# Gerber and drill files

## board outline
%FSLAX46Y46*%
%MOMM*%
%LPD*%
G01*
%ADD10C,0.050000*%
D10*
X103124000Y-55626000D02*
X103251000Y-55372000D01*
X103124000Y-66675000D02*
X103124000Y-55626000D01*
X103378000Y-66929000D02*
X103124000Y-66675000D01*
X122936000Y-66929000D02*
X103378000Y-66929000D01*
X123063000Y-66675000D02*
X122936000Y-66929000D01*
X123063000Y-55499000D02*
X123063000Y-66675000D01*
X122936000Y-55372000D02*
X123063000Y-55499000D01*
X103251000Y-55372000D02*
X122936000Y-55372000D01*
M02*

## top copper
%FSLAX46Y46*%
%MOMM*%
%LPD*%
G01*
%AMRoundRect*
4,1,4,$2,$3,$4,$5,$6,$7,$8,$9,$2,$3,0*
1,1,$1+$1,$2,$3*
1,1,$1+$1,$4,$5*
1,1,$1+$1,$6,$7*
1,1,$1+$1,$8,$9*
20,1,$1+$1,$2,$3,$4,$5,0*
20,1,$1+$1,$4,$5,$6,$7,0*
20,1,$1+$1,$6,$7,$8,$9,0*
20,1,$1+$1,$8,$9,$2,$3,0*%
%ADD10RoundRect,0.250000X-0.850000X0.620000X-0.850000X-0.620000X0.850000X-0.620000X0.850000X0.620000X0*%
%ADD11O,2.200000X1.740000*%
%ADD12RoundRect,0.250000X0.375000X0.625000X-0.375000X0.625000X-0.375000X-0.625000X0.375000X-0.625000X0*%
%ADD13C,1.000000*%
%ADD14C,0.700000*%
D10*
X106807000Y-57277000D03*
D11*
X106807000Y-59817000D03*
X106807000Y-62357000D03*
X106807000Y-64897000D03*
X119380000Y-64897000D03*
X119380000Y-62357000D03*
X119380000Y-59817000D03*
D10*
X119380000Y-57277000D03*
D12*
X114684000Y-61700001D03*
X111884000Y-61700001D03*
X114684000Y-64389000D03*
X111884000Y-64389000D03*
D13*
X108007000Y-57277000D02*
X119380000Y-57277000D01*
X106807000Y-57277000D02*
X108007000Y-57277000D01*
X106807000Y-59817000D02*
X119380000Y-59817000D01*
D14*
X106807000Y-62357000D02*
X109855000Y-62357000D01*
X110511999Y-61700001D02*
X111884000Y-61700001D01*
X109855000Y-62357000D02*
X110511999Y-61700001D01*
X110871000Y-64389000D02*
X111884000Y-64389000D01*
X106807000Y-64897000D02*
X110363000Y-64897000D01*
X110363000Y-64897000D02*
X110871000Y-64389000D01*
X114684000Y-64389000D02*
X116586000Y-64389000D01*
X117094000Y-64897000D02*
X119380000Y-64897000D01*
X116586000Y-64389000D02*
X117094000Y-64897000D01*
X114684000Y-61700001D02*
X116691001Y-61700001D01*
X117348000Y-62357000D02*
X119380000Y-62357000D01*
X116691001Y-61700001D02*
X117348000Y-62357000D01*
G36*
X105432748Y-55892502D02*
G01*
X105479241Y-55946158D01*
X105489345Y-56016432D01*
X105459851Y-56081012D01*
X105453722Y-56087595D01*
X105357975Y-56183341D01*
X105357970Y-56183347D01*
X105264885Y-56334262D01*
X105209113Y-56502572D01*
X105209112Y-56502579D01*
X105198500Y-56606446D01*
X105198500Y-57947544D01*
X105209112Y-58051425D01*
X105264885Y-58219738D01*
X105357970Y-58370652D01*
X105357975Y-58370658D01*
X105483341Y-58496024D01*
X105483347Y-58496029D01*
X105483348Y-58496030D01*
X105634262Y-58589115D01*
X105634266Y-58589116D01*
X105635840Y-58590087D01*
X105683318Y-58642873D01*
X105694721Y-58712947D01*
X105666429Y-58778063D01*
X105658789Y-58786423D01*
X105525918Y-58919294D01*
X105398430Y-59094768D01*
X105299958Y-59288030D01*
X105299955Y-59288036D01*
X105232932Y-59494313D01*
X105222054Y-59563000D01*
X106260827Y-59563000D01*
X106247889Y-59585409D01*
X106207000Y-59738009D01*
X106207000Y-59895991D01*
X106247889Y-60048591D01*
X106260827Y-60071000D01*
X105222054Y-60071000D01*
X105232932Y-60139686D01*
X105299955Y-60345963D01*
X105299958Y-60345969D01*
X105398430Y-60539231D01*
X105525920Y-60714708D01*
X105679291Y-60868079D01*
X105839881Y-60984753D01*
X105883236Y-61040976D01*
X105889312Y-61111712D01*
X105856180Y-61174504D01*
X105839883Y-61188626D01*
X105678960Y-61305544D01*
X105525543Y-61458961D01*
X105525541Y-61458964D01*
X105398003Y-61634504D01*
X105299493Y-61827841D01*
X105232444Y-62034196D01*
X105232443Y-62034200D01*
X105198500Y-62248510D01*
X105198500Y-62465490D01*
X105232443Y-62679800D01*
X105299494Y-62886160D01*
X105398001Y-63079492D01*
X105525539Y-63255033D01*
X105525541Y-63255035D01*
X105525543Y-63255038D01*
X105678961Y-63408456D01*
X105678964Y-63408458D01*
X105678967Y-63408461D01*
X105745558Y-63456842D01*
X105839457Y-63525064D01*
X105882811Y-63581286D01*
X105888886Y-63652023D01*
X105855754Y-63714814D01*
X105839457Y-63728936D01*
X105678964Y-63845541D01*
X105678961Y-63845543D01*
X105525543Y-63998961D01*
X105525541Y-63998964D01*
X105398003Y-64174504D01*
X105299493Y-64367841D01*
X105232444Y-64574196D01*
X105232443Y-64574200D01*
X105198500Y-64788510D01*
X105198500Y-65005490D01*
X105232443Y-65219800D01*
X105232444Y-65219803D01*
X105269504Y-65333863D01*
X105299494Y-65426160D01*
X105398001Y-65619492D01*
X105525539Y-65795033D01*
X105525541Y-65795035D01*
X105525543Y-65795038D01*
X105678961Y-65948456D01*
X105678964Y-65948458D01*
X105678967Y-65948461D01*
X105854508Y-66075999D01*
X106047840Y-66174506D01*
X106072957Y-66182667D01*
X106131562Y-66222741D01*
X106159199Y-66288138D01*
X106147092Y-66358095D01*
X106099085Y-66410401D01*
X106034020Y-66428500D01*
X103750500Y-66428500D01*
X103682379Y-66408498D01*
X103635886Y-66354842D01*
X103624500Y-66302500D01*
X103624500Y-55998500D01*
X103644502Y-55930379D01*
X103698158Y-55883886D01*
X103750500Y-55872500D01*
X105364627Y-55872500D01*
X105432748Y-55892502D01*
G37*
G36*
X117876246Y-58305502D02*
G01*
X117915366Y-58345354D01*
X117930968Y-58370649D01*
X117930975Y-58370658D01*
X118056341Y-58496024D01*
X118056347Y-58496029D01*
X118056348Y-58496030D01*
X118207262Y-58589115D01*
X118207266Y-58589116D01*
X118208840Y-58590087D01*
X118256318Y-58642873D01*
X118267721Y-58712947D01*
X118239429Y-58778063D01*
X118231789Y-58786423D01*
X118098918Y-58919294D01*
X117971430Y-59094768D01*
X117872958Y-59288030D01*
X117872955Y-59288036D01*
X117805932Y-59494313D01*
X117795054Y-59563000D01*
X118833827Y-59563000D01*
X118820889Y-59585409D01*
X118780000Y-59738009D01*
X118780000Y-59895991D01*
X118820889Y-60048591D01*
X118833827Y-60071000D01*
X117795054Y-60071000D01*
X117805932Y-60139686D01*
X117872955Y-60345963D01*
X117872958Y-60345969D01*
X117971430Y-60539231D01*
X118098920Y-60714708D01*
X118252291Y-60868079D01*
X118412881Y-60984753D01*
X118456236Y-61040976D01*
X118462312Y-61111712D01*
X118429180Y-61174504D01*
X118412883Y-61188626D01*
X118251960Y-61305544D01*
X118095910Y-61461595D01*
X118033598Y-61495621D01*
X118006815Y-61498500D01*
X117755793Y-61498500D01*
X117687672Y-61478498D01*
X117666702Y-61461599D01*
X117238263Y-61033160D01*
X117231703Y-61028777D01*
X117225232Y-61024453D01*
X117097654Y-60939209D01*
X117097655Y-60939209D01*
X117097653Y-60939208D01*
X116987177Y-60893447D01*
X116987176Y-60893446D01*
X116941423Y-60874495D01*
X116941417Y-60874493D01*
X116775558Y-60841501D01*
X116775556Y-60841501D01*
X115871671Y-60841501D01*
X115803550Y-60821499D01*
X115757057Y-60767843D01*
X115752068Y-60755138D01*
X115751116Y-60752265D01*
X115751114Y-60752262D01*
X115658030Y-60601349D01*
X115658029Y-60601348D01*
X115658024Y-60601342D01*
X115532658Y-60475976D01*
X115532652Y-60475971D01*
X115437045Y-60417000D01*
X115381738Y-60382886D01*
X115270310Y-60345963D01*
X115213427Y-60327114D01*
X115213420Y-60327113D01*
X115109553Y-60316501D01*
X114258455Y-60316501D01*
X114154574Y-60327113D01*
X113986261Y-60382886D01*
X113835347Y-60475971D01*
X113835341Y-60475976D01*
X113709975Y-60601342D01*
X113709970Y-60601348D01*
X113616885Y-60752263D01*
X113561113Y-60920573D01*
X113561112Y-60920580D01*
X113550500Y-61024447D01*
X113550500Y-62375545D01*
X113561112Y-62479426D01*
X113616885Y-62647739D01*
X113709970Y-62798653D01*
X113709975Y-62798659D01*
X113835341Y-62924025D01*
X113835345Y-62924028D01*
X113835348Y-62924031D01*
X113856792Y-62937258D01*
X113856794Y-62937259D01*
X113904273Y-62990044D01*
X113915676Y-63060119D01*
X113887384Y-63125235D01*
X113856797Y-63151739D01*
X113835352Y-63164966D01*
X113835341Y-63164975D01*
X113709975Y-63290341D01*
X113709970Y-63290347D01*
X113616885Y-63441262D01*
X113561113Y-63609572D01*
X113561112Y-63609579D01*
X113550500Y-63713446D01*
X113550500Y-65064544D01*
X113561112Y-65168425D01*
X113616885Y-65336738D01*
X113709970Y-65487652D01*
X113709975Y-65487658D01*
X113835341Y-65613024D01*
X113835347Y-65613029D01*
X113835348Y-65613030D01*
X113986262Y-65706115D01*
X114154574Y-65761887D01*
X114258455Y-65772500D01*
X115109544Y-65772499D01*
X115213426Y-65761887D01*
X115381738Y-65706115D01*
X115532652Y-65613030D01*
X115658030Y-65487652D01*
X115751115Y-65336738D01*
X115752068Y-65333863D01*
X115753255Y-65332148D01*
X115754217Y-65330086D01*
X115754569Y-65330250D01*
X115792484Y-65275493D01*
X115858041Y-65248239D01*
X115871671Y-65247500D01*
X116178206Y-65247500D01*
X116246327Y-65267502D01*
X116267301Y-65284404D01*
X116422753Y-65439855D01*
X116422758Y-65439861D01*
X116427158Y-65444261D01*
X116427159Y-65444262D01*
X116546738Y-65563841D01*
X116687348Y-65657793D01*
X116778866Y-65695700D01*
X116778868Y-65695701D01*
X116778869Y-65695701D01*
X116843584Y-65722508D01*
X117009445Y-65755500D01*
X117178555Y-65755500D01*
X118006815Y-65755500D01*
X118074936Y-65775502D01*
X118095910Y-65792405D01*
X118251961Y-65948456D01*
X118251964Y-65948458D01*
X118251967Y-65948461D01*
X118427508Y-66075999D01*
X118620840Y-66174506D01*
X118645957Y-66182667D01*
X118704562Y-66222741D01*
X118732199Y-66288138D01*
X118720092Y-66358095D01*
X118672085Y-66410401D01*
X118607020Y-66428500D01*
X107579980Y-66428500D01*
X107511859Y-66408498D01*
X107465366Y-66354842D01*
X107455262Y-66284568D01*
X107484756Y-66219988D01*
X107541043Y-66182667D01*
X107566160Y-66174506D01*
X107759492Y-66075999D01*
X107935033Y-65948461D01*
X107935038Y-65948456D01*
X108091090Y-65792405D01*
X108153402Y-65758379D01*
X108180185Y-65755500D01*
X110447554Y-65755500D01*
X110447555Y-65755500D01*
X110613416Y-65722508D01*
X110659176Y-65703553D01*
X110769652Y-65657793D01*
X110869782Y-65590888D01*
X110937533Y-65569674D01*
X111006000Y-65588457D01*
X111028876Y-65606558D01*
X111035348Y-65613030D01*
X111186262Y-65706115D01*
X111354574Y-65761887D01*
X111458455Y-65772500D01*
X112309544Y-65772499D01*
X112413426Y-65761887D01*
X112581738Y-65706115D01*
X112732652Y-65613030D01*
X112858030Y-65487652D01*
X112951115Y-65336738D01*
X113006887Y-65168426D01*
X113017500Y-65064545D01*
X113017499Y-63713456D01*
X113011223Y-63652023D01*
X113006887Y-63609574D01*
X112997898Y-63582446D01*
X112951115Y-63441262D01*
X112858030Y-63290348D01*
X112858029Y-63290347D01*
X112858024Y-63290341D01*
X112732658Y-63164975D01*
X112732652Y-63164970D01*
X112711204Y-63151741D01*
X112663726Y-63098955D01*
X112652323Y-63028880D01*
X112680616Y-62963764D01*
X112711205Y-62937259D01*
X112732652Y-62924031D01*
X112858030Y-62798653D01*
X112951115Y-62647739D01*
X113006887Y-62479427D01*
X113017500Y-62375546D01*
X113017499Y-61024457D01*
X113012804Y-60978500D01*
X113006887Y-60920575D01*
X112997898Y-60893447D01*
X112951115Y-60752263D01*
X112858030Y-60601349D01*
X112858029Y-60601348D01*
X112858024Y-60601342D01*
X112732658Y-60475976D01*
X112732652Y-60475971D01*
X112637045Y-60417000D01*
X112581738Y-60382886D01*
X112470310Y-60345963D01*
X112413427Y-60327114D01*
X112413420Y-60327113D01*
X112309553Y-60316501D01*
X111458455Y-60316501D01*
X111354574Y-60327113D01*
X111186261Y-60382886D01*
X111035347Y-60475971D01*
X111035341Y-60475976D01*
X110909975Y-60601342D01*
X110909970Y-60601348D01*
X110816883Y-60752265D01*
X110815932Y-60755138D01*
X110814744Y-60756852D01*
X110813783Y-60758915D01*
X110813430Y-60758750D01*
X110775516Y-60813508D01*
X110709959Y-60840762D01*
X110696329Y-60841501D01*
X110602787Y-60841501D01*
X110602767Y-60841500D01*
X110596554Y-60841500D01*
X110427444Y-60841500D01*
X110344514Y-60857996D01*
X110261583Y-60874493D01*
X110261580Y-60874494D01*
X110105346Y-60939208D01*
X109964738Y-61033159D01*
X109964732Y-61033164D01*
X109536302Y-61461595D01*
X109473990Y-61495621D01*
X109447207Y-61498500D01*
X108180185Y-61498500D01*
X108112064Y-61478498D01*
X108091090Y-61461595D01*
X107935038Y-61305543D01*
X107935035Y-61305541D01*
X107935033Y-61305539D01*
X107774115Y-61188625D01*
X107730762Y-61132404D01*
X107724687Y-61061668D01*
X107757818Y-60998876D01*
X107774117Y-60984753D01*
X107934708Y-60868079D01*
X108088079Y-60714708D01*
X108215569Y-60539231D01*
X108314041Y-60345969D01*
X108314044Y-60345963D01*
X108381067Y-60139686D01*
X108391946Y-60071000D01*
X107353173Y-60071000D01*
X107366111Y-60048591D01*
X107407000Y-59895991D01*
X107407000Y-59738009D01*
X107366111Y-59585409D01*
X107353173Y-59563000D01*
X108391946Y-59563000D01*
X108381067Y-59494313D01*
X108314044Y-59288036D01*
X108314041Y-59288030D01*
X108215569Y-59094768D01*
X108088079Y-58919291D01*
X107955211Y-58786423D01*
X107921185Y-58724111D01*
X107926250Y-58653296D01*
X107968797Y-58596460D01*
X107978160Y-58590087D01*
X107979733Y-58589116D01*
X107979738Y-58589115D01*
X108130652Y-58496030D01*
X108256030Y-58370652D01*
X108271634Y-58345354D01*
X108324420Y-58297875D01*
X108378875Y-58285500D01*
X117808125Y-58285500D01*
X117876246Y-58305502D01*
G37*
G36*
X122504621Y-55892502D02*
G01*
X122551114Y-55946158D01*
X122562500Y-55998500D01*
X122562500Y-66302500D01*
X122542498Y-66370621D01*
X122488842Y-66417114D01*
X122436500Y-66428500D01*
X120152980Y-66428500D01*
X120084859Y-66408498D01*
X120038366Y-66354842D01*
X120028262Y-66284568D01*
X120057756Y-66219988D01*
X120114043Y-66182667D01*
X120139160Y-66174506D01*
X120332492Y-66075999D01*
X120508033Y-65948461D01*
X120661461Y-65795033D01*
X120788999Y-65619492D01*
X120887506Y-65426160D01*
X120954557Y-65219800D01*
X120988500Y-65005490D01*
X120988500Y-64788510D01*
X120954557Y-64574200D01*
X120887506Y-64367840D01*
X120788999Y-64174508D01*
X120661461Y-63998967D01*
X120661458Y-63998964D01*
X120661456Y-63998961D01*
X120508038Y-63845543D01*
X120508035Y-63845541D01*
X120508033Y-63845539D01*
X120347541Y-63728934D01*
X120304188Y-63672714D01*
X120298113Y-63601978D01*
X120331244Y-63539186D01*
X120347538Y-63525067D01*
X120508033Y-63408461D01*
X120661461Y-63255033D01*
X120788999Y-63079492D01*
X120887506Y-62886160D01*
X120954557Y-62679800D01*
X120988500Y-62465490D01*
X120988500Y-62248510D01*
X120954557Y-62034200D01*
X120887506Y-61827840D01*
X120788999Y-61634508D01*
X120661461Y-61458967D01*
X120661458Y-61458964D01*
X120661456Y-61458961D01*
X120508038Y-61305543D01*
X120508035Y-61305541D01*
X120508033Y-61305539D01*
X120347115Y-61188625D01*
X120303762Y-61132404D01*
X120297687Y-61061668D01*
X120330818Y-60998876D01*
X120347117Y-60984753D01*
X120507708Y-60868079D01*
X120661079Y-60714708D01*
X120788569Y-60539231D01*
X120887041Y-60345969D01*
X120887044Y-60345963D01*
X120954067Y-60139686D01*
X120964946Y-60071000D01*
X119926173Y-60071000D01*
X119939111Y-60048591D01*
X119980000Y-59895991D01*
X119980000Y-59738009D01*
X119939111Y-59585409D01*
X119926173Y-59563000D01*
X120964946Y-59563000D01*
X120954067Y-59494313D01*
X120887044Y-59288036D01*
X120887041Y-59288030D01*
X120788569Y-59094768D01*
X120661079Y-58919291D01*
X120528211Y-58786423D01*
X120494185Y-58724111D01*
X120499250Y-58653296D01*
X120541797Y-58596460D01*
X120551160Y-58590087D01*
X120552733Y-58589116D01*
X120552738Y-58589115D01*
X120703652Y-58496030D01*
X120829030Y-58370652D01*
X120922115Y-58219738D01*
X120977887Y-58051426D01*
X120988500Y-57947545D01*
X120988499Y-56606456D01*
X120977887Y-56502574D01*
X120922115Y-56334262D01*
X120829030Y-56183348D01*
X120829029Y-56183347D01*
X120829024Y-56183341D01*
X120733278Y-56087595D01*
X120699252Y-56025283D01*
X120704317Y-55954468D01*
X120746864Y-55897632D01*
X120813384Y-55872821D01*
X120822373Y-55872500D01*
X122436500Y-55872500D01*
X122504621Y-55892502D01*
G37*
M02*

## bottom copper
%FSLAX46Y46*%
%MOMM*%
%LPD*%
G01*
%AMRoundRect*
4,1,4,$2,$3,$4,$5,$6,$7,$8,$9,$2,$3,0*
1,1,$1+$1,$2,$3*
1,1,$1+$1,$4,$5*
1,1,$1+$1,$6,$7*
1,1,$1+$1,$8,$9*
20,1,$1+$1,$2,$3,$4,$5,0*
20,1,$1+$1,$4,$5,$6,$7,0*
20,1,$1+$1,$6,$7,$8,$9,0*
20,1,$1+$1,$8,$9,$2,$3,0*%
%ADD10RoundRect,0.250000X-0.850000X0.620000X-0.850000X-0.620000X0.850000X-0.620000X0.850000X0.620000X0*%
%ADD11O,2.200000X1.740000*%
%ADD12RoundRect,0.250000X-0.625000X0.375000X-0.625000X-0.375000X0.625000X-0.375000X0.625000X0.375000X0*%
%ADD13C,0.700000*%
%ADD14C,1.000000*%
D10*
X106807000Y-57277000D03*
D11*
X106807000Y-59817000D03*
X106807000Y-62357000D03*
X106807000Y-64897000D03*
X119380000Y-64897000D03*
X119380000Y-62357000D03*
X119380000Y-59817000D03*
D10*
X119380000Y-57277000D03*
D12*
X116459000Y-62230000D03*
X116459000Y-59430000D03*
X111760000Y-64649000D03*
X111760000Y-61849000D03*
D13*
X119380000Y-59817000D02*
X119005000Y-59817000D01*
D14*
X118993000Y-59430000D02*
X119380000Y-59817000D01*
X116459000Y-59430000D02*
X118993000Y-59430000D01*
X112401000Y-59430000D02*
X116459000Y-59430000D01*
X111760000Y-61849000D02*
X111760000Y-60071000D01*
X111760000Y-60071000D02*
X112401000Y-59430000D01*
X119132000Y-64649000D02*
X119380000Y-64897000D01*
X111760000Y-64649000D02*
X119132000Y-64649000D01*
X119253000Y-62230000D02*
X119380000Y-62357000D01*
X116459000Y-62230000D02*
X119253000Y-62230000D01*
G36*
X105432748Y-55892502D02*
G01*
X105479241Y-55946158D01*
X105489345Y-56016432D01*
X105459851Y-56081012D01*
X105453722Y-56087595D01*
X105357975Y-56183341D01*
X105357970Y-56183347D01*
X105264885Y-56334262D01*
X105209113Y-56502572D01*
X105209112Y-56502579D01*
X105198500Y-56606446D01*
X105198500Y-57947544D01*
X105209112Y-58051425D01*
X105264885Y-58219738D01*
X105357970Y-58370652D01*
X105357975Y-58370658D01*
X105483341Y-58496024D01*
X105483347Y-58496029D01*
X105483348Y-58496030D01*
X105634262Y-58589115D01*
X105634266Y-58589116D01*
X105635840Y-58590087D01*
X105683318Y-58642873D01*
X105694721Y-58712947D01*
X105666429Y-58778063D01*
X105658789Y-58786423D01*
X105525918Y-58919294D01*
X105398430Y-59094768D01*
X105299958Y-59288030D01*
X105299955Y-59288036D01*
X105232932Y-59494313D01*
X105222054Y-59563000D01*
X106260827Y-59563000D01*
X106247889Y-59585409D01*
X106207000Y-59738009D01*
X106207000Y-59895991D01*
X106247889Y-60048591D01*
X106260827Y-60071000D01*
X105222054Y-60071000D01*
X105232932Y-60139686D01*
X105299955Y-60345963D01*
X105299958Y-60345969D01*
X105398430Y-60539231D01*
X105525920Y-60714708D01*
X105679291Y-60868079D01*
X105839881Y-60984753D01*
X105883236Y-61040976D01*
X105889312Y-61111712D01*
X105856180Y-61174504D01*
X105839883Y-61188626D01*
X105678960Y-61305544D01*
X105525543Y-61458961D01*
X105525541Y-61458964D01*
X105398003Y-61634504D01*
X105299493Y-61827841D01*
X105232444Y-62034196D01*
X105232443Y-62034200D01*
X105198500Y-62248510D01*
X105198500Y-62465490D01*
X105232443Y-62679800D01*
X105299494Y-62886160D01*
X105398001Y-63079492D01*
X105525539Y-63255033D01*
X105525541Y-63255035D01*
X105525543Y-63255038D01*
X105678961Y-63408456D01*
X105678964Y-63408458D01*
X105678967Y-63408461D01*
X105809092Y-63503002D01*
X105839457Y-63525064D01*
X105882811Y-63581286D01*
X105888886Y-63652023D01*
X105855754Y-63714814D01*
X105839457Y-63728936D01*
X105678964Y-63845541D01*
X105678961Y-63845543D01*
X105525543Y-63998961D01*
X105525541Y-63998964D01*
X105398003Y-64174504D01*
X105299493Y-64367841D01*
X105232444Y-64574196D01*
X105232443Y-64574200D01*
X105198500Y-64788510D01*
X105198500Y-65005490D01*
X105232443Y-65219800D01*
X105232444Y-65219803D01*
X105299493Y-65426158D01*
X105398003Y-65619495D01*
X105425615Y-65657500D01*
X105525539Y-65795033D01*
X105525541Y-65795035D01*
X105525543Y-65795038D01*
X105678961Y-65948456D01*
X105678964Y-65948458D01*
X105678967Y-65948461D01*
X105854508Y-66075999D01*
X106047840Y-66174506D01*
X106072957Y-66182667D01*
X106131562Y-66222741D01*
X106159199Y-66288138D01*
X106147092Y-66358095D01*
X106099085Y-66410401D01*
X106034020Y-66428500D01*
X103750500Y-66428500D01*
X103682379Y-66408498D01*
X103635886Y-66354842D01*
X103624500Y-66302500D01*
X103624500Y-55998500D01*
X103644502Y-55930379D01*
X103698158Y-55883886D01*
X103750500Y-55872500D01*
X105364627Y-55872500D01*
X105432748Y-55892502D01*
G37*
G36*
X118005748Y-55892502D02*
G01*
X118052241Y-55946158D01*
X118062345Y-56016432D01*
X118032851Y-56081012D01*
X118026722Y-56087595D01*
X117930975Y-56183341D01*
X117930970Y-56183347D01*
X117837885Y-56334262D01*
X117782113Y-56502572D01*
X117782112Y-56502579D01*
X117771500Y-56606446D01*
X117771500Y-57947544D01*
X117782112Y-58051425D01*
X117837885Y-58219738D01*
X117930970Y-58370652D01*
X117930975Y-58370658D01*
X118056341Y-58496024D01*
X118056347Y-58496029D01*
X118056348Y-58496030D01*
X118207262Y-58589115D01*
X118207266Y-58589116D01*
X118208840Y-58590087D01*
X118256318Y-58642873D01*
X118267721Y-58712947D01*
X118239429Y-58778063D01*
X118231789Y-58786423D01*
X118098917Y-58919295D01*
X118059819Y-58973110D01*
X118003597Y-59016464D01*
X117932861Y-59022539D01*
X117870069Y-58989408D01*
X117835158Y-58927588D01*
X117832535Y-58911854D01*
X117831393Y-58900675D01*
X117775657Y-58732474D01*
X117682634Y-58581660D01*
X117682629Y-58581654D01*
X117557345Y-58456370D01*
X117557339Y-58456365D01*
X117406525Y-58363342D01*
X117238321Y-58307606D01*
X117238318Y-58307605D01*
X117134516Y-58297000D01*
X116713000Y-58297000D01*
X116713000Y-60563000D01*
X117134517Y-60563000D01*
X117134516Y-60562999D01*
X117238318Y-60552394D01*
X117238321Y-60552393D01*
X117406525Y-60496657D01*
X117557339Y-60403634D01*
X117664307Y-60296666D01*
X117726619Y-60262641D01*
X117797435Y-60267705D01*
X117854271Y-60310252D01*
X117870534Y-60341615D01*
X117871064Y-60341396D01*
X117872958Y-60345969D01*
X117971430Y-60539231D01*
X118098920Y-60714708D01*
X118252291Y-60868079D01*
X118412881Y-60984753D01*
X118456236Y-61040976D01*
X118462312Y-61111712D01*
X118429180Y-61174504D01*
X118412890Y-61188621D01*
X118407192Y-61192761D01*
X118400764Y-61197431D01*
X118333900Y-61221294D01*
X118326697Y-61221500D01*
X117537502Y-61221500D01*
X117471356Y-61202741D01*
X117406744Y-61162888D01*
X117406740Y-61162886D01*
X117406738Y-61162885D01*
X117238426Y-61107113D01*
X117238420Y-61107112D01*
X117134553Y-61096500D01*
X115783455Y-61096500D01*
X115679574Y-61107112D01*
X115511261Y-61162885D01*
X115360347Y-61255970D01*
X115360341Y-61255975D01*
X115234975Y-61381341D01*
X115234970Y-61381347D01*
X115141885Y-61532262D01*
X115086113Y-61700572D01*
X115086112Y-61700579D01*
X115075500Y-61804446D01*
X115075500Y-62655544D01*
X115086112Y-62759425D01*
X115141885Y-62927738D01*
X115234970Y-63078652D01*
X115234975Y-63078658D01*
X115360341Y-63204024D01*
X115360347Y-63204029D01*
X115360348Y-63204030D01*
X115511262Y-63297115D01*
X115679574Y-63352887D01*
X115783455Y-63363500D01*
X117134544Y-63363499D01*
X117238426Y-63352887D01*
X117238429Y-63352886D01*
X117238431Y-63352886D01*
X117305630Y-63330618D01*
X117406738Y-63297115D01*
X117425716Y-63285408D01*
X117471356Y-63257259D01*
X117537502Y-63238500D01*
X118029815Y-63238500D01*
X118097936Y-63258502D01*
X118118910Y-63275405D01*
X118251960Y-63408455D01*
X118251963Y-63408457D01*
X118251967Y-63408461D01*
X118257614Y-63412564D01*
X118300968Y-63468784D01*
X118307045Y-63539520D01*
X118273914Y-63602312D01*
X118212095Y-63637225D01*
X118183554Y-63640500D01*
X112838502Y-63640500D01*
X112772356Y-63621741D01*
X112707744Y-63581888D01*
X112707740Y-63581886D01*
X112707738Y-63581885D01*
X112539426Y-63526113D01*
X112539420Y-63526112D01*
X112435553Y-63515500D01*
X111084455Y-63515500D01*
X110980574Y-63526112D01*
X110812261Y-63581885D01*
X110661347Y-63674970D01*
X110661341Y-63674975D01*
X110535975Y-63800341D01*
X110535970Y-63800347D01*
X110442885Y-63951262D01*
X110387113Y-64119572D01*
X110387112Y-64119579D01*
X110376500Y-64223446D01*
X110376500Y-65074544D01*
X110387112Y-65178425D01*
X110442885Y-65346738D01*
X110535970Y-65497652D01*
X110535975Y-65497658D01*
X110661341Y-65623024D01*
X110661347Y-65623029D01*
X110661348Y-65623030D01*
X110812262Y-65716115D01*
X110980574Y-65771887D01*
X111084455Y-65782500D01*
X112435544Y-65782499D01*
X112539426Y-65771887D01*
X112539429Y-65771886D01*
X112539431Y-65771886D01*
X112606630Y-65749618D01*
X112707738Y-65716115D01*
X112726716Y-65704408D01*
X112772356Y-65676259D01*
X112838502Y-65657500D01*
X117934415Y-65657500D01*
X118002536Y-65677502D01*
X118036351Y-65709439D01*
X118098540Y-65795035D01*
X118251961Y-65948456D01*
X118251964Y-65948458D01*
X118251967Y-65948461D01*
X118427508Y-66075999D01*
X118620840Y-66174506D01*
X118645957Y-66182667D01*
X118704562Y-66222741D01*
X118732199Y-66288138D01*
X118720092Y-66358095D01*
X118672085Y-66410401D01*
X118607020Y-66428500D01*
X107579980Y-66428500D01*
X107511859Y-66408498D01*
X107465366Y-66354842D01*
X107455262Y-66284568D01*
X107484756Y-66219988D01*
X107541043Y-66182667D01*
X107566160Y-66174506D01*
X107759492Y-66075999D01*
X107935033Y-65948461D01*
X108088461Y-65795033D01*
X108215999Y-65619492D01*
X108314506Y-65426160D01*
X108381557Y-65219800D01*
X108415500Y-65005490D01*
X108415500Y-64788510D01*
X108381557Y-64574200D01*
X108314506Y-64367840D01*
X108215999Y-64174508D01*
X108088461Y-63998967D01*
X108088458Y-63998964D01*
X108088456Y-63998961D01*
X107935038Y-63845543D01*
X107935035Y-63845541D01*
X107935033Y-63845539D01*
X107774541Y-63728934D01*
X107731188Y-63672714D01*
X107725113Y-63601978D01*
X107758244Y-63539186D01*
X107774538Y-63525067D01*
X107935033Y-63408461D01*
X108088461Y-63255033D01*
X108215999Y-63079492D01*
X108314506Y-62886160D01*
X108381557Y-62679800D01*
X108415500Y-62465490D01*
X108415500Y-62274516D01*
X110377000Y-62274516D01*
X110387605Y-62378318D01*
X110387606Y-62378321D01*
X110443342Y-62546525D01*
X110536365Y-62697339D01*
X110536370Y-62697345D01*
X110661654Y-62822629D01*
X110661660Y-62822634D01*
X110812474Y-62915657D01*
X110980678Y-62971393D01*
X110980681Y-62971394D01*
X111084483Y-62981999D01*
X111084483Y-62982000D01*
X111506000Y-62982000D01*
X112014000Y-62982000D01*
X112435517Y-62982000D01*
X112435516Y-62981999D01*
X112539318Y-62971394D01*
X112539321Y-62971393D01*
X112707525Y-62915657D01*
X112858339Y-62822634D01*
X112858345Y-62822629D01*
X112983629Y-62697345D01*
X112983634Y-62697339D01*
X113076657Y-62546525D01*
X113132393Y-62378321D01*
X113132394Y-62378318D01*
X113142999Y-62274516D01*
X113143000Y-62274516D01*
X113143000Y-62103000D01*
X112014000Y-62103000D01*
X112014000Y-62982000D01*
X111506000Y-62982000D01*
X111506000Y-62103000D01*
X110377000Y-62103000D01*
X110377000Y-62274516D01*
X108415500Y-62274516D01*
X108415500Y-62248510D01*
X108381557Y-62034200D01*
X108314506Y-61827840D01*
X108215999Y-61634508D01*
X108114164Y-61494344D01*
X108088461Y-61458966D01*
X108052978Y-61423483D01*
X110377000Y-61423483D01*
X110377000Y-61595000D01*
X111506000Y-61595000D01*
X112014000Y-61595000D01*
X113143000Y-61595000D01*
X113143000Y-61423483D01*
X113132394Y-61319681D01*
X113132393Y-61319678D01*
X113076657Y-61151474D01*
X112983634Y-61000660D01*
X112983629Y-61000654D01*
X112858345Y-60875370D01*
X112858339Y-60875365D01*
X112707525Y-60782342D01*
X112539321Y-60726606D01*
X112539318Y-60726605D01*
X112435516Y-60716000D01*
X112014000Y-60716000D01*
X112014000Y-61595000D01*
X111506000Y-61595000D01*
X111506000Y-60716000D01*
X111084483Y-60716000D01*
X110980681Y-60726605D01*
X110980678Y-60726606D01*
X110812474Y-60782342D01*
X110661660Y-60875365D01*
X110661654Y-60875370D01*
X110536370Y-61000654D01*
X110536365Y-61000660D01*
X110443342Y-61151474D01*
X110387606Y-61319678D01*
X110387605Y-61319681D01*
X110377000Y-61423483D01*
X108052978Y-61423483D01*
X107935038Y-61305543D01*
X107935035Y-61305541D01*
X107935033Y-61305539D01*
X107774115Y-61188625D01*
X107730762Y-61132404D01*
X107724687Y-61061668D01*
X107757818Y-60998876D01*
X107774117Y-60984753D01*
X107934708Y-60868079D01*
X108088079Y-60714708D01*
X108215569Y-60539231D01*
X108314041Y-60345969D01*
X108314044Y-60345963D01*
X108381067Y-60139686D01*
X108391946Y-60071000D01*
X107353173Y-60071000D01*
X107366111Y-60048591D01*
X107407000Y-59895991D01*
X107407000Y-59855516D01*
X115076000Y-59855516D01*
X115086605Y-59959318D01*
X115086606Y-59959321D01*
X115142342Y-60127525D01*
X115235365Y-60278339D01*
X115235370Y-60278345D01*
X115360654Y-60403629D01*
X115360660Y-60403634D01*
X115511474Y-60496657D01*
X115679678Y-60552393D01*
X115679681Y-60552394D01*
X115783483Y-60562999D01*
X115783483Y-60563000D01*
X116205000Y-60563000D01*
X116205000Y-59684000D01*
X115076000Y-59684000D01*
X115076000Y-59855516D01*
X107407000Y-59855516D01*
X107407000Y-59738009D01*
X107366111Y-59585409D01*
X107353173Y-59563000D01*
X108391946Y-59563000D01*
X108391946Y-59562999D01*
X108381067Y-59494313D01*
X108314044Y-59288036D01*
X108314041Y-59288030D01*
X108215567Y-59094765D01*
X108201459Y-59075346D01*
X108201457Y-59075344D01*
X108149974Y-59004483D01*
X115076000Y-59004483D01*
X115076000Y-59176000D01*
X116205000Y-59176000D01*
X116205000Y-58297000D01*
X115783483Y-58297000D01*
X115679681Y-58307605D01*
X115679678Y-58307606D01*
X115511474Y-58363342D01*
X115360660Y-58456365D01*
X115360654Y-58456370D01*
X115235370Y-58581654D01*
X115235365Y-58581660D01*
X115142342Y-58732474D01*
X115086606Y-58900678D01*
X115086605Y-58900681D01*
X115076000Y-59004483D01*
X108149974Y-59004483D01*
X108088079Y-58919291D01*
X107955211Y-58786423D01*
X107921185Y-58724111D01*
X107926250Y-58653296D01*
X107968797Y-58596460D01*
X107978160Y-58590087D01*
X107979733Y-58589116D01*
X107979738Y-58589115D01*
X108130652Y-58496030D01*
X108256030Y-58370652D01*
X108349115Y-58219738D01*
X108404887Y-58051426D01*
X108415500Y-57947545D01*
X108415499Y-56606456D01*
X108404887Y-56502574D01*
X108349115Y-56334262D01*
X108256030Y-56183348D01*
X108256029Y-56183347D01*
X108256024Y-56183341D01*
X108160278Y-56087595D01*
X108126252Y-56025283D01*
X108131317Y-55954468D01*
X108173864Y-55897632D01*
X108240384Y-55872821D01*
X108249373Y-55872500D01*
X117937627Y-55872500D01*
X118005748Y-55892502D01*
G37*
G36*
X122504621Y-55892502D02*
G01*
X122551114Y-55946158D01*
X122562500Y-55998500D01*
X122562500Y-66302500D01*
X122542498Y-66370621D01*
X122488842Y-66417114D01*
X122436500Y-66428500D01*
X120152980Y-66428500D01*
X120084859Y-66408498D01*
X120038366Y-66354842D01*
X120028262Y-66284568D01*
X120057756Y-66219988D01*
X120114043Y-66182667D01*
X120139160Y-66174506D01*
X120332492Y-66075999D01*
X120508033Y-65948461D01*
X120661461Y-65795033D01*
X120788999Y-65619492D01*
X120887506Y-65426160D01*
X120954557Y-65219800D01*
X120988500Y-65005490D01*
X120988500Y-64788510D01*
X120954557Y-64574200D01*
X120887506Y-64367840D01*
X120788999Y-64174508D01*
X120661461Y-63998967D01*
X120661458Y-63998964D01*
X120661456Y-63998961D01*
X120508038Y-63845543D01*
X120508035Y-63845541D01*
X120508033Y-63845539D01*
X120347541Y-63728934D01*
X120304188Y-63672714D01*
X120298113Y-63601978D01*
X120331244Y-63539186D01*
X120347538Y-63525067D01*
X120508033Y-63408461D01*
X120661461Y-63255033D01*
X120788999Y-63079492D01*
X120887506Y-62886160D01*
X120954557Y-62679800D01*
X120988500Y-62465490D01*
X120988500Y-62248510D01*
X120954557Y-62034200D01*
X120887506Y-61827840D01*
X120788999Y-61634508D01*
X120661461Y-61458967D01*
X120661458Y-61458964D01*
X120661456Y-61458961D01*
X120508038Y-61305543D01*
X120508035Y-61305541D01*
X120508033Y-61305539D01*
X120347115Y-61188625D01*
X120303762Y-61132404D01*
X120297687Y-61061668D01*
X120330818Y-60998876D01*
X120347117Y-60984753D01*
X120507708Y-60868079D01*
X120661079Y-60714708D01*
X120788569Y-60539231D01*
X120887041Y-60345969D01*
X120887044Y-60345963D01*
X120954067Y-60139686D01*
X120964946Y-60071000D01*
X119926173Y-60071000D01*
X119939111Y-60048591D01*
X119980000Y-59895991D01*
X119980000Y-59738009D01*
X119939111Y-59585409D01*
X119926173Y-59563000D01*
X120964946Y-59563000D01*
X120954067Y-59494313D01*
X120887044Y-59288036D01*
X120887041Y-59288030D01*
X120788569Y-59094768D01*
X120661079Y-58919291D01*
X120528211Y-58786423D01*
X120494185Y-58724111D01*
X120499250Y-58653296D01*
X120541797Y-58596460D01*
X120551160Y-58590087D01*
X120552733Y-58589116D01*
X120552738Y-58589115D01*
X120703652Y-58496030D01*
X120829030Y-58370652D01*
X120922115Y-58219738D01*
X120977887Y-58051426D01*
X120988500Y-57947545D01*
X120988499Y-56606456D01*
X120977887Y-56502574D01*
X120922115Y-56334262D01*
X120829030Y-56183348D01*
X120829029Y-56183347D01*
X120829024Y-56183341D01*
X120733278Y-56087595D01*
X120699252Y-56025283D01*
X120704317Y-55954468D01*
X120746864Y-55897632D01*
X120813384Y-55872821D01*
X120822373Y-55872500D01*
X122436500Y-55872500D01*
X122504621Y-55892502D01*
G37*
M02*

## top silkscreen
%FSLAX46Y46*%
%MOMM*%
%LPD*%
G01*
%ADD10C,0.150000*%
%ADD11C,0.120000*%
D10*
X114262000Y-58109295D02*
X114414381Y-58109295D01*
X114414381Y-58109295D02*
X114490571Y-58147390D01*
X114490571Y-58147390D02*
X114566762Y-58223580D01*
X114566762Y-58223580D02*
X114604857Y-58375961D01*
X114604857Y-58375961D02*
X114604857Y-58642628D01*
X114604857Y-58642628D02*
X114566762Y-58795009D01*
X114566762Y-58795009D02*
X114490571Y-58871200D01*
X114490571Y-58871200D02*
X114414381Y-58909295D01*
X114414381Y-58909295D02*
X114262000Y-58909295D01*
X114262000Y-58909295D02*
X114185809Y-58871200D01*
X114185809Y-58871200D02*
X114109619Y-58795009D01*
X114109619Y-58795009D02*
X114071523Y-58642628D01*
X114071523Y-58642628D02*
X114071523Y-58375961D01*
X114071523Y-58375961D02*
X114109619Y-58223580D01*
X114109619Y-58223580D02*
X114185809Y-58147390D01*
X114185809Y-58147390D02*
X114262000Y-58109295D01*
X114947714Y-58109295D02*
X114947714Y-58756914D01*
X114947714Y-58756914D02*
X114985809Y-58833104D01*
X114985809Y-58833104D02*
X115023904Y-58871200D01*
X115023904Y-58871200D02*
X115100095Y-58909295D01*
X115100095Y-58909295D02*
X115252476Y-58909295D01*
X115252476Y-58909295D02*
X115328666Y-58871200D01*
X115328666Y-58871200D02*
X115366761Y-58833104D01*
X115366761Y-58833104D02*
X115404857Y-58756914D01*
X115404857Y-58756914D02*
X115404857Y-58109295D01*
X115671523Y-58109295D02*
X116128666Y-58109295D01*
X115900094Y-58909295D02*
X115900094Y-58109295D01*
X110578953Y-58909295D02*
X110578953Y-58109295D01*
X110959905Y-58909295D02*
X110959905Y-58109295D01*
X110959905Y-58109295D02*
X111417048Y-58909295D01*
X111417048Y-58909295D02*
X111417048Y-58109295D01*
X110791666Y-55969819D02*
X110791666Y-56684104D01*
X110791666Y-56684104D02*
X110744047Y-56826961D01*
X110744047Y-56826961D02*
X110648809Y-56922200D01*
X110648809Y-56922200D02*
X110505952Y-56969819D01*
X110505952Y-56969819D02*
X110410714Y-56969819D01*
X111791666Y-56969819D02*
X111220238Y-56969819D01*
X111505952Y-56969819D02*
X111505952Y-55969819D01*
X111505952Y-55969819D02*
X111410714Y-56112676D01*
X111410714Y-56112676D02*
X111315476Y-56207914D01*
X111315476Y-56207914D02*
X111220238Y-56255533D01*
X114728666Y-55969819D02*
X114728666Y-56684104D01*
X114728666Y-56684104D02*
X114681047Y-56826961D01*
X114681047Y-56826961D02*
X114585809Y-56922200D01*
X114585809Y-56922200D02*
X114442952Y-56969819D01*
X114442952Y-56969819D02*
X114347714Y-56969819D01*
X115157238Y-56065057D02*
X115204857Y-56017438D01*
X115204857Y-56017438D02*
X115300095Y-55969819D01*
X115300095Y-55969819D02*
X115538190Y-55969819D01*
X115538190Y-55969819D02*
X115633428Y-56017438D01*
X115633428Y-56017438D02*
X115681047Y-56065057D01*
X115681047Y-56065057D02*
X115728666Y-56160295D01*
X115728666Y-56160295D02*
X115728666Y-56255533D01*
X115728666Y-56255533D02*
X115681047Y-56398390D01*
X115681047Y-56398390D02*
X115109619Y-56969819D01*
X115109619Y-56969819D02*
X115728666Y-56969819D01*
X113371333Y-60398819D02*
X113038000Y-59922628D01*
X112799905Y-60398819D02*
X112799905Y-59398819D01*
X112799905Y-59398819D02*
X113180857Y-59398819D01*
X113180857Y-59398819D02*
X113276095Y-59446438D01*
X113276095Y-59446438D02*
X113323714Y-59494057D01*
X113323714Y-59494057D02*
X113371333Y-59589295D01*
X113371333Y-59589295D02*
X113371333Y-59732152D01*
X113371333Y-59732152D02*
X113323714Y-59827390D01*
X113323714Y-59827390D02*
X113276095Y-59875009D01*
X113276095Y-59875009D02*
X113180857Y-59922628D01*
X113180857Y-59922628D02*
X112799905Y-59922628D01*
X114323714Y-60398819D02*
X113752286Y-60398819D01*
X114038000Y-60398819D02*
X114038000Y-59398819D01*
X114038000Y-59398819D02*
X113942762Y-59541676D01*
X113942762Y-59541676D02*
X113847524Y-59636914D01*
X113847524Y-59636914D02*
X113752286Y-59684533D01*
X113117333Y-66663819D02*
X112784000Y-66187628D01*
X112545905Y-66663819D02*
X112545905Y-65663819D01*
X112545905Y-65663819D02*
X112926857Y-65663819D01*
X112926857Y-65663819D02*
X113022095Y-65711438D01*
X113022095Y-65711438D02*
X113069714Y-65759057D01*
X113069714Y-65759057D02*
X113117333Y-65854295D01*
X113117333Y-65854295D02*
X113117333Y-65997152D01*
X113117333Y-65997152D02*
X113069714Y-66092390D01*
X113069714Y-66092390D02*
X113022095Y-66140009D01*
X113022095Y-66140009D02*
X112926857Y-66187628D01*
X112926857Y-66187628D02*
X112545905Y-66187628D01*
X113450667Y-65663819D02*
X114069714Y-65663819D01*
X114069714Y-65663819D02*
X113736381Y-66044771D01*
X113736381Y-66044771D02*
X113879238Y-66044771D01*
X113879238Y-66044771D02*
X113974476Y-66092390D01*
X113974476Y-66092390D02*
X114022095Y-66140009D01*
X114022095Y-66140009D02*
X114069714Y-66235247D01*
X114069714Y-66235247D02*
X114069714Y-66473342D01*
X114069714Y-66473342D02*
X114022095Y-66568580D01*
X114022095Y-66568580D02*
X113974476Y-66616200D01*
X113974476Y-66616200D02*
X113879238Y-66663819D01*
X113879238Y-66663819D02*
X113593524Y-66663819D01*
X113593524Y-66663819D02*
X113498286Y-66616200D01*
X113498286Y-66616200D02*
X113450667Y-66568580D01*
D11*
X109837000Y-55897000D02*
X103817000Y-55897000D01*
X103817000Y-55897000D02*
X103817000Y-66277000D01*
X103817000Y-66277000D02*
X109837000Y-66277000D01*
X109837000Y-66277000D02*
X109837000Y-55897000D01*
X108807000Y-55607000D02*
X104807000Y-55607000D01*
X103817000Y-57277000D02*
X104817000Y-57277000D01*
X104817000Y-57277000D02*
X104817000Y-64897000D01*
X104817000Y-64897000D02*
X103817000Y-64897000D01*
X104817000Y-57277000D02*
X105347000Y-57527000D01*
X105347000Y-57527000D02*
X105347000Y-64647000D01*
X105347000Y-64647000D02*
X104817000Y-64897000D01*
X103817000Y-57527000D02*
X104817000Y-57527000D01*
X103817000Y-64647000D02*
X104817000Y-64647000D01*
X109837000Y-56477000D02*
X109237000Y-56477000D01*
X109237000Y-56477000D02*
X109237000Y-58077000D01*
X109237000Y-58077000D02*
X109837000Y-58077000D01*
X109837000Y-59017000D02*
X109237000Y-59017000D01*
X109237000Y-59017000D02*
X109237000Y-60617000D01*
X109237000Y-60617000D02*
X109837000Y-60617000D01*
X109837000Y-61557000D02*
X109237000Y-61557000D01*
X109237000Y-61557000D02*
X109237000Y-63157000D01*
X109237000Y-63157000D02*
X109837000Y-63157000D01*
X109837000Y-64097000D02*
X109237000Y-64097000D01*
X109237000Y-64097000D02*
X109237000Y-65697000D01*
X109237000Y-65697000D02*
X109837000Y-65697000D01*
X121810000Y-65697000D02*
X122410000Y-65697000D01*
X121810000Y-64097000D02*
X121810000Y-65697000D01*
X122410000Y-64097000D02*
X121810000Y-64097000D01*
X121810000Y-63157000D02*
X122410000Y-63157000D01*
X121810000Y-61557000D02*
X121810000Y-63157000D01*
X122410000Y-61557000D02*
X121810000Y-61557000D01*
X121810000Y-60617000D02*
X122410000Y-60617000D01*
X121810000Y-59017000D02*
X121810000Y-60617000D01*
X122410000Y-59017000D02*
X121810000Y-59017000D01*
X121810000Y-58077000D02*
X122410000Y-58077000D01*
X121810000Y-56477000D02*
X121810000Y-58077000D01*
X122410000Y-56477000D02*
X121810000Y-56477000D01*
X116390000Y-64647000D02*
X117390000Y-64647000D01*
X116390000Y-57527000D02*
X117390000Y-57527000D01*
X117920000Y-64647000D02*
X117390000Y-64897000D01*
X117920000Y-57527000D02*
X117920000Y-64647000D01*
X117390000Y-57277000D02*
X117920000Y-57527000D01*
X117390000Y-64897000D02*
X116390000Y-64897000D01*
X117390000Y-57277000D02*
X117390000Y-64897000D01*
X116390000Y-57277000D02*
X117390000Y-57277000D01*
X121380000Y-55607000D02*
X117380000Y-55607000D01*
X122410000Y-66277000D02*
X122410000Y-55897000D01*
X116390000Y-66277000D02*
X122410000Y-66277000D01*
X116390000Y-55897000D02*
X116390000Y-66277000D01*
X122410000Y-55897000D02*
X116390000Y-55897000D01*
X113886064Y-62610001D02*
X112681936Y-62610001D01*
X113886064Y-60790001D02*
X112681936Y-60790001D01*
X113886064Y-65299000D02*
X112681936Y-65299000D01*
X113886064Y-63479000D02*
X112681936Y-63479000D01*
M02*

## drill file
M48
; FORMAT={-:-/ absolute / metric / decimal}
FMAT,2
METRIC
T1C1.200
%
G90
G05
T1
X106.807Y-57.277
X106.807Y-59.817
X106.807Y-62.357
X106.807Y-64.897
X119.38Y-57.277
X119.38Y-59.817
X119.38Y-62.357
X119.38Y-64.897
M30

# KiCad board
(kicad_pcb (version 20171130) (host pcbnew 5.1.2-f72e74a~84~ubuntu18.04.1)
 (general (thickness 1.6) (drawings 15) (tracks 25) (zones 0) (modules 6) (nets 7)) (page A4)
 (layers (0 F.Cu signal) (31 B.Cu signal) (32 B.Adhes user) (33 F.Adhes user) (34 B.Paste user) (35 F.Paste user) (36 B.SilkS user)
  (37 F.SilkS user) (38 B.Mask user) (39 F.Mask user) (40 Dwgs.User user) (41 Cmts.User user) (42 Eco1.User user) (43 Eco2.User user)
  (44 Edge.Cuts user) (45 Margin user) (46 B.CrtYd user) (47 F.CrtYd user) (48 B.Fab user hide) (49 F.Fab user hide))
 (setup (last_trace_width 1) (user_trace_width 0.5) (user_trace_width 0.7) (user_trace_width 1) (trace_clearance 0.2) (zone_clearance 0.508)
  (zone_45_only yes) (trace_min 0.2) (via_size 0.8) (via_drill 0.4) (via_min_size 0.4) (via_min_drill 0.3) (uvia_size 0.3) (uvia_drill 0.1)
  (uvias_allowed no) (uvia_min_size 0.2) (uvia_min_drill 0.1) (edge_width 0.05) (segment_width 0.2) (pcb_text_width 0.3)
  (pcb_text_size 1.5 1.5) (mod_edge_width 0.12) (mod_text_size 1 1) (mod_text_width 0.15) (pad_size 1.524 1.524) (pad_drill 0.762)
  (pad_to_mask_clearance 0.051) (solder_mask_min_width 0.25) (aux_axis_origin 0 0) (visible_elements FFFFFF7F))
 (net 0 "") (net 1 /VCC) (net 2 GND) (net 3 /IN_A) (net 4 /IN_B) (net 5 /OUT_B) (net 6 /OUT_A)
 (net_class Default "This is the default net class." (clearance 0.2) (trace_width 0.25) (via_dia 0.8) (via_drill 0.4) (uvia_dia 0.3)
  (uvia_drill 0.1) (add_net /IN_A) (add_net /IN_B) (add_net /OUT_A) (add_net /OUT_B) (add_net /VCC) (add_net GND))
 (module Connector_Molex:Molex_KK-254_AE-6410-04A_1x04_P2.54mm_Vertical (layer F.Cu) (at 106.807 57.277 270)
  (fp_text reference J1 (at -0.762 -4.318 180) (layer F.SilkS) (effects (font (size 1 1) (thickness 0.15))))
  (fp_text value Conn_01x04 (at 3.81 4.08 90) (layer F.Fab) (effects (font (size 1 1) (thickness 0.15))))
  (fp_line (start -1.38 -3.03) (end -1.38 2.99) (layer F.SilkS) (width 0.12))
  (fp_line (start -1.38 2.99) (end 9 2.99) (layer F.SilkS) (width 0.12))
  (fp_line (start 9 2.99) (end 9 -3.03) (layer F.SilkS) (width 0.12))
  (fp_line (start 9 -3.03) (end -1.38 -3.03) (layer F.SilkS) (width 0.12))
  (fp_line (start -1.67 -2) (end -1.67 2) (layer F.SilkS) (width 0.12))
  (fp_line (start 0 2.99) (end 0 1.99) (layer F.SilkS) (width 0.12))
  (fp_line (start 0 1.99) (end 7.62 1.99) (layer F.SilkS) (width 0.12))
  (fp_line (start 7.62 1.99) (end 7.62 2.99) (layer F.SilkS) (width 0.12))
  (fp_line (start 0 1.99) (end 0.25 1.46) (layer F.SilkS) (width 0.12))
  (fp_line (start 0.25 1.46) (end 7.37 1.46) (layer F.SilkS) (width 0.12))
  (fp_line (start 7.37 1.46) (end 7.62 1.99) (layer F.SilkS) (width 0.12))
  (fp_line (start 0.25 2.99) (end 0.25 1.99) (layer F.SilkS) (width 0.12))
  (fp_line (start 7.37 2.99) (end 7.37 1.99) (layer F.SilkS) (width 0.12))
  (fp_line (start -0.8 -3.03) (end -0.8 -2.43) (layer F.SilkS) (width 0.12))
  (fp_line (start -0.8 -2.43) (end 0.8 -2.43) (layer F.SilkS) (width 0.12))
  (fp_line (start 0.8 -2.43) (end 0.8 -3.03) (layer F.SilkS) (width 0.12))
  (fp_line (start 1.74 -3.03) (end 1.74 -2.43) (layer F.SilkS) (width 0.12))
  (fp_line (start 1.74 -2.43) (end 3.34 -2.43) (layer F.SilkS) (width 0.12))
  (fp_line (start 3.34 -2.43) (end 3.34 -3.03) (layer F.SilkS) (width 0.12))
  (fp_line (start 4.28 -3.03) (end 4.28 -2.43) (layer F.SilkS) (width 0.12))
  (fp_line (start 4.28 -2.43) (end 5.88 -2.43) (layer F.SilkS) (width 0.12))
  (fp_line (start 5.88 -2.43) (end 5.88 -3.03) (layer F.SilkS) (width 0.12))
  (fp_line (start 6.82 -3.03) (end 6.82 -2.43) (layer F.SilkS) (width 0.12))
  (fp_line (start 6.82 -2.43) (end 8.42 -2.43) (layer F.SilkS) (width 0.12))
  (fp_line (start 8.42 -2.43) (end 8.42 -3.03) (layer F.SilkS) (width 0.12))
  (pad 1 thru_hole roundrect (at 0 0 270) (size 1.74 2.2) (drill 1.2) (layers *.Cu *.Mask) (roundrect_rratio 0.143678) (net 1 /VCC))
  (pad 2 thru_hole oval (at 2.54 0 270) (size 1.74 2.2) (drill 1.2) (layers *.Cu *.Mask) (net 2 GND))
  (pad 3 thru_hole oval (at 5.08 0 270) (size 1.74 2.2) (drill 1.2) (layers *.Cu *.Mask) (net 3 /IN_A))
  (pad 4 thru_hole oval (at 7.62 0 270) (size 1.74 2.2) (drill 1.2) (layers *.Cu *.Mask) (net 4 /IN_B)))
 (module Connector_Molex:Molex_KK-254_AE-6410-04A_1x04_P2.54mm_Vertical (layer F.Cu) (at 119.38 57.277 270)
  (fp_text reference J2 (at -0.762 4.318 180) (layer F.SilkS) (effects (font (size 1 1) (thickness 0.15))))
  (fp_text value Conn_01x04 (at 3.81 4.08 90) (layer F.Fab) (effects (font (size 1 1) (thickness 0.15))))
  (fp_line (start 8.42 -2.43) (end 8.42 -3.03) (layer F.SilkS) (width 0.12))
  (fp_line (start 6.82 -2.43) (end 8.42 -2.43) (layer F.SilkS) (width 0.12))
  (fp_line (start 6.82 -3.03) (end 6.82 -2.43) (layer F.SilkS) (width 0.12))
  (fp_line (start 5.88 -2.43) (end 5.88 -3.03) (layer F.SilkS) (width 0.12))
  (fp_line (start 4.28 -2.43) (end 5.88 -2.43) (layer F.SilkS) (width 0.12))
  (fp_line (start 4.28 -3.03) (end 4.28 -2.43) (layer F.SilkS) (width 0.12))
  (fp_line (start 3.34 -2.43) (end 3.34 -3.03) (layer F.SilkS) (width 0.12))
  (fp_line (start 1.74 -2.43) (end 3.34 -2.43) (layer F.SilkS) (width 0.12))
  (fp_line (start 1.74 -3.03) (end 1.74 -2.43) (layer F.SilkS) (width 0.12))
  (fp_line (start 0.8 -2.43) (end 0.8 -3.03) (layer F.SilkS) (width 0.12))
  (fp_line (start -0.8 -2.43) (end 0.8 -2.43) (layer F.SilkS) (width 0.12))
  (fp_line (start -0.8 -3.03) (end -0.8 -2.43) (layer F.SilkS) (width 0.12))
  (fp_line (start 7.37 2.99) (end 7.37 1.99) (layer F.SilkS) (width 0.12))
  (fp_line (start 0.25 2.99) (end 0.25 1.99) (layer F.SilkS) (width 0.12))
  (fp_line (start 7.37 1.46) (end 7.62 1.99) (layer F.SilkS) (width 0.12))
  (fp_line (start 0.25 1.46) (end 7.37 1.46) (layer F.SilkS) (width 0.12))
  (fp_line (start 0 1.99) (end 0.25 1.46) (layer F.SilkS) (width 0.12))
  (fp_line (start 7.62 1.99) (end 7.62 2.99) (layer F.SilkS) (width 0.12))
  (fp_line (start 0 1.99) (end 7.62 1.99) (layer F.SilkS) (width 0.12))
  (fp_line (start 0 2.99) (end 0 1.99) (layer F.SilkS) (width 0.12))
  (fp_line (start -1.67 -2) (end -1.67 2) (layer F.SilkS) (width 0.12))
  (fp_line (start 9 -3.03) (end -1.38 -3.03) (layer F.SilkS) (width 0.12))
  (fp_line (start 9 2.99) (end 9 -3.03) (layer F.SilkS) (width 0.12))
  (fp_line (start -1.38 2.99) (end 9 2.99) (layer F.SilkS) (width 0.12))
  (fp_line (start -1.38 -3.03) (end -1.38 2.99) (layer F.SilkS) (width 0.12))
  (pad 4 thru_hole oval (at 7.62 0 270) (size 1.74 2.2) (drill 1.2) (layers *.Cu *.Mask) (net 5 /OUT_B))
  (pad 3 thru_hole oval (at 5.08 0 270) (size 1.74 2.2) (drill 1.2) (layers *.Cu *.Mask) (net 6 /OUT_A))
  (pad 2 thru_hole oval (at 2.54 0 270) (size 1.74 2.2) (drill 1.2) (layers *.Cu *.Mask) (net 2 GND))
  (pad 1 thru_hole roundrect (at 0 0 270) (size 1.74 2.2) (drill 1.2) (layers *.Cu *.Mask) (roundrect_rratio 0.143678) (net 1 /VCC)))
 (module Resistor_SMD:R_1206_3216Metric (layer F.Cu) (at 113.284 61.700001 180)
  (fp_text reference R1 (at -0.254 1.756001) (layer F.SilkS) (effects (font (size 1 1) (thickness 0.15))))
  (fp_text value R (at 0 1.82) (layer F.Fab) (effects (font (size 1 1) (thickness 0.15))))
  (fp_line (start -0.602064 -0.91) (end 0.602064 -0.91) (layer F.SilkS) (width 0.12))
  (fp_line (start -0.602064 0.91) (end 0.602064 0.91) (layer F.SilkS) (width 0.12))
  (pad 1 smd roundrect (at -1.4 0 180) (size 1.25 1.75) (layers F.Cu F.Paste F.Mask) (roundrect_rratio 0.2) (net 6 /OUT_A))
  (pad 2 smd roundrect (at 1.4 0 180) (size 1.25 1.75) (layers F.Cu F.Paste F.Mask) (roundrect_rratio 0.2) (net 3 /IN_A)))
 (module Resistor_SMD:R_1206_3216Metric (layer B.Cu) (at 116.459 60.83 270)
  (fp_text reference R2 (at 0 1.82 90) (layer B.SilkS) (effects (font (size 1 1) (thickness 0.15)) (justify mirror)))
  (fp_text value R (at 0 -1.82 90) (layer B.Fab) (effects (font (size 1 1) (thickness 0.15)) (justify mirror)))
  (pad 2 smd roundrect (at 1.4 0 270) (size 1.25 1.75) (layers B.Cu B.Paste B.Mask) (roundrect_rratio 0.2) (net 6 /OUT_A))
  (pad 1 smd roundrect (at -1.4 0 270) (size 1.25 1.75) (layers B.Cu B.Paste B.Mask) (roundrect_rratio 0.2) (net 2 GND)))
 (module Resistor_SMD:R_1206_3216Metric (layer F.Cu) (at 113.284 64.389 180)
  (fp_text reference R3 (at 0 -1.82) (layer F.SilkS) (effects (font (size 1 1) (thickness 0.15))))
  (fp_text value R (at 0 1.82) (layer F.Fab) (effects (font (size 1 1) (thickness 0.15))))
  (fp_line (start -0.602064 -0.91) (end 0.602064 -0.91) (layer F.SilkS) (width 0.12))
  (fp_line (start -0.602064 0.91) (end 0.602064 0.91) (layer F.SilkS) (width 0.12))
  (pad 1 smd roundrect (at -1.4 0 180) (size 1.25 1.75) (layers F.Cu F.Paste F.Mask) (roundrect_rratio 0.2) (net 5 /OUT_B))
  (pad 2 smd roundrect (at 1.4 0 180) (size 1.25 1.75) (layers F.Cu F.Paste F.Mask) (roundrect_rratio 0.2) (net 4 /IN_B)))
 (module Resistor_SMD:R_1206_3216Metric (layer B.Cu) (at 111.76 63.249 270)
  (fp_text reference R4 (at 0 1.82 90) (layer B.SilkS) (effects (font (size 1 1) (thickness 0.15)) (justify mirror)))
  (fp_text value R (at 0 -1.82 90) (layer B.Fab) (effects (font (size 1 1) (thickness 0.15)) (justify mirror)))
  (pad 2 smd roundrect (at 1.4 0 270) (size 1.25 1.75) (layers B.Cu B.Paste B.Mask) (roundrect_rratio 0.2) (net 5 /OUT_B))
  (pad 1 smd roundrect (at -1.4 0 270) (size 1.25 1.75) (layers B.Cu B.Paste B.Mask) (roundrect_rratio 0.2) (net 2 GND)))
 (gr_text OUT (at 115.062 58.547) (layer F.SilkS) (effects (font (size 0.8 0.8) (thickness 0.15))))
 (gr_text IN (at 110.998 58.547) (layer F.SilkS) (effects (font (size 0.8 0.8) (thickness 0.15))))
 (gr_line (start 103.124 55.626) (end 103.251 55.372) (layer Edge.Cuts) (width 0.05))
 (gr_line (start 103.124 66.675) (end 103.124 55.626) (layer Edge.Cuts) (width 0.05))
 (gr_line (start 103.378 66.929) (end 103.124 66.675) (layer Edge.Cuts) (width 0.05))
 (gr_line (start 122.936 66.929) (end 103.378 66.929) (layer Edge.Cuts) (width 0.05))
 (gr_line (start 123.063 66.675) (end 122.936 66.929) (layer Edge.Cuts) (width 0.05))
 (gr_line (start 123.063 55.499) (end 123.063 66.675) (layer Edge.Cuts) (width 0.05))
 (gr_line (start 122.936 55.372) (end 123.063 55.499) (layer Edge.Cuts) (width 0.05))
 (gr_line (start 103.251 55.372) (end 122.936 55.372) (layer Edge.Cuts) (width 0.05))
 (segment (start 108.007 57.277) (end 119.38 57.277) (width 1) (layer F.Cu) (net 1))
 (segment (start 106.807 57.277) (end 108.007 57.277) (width 1) (layer F.Cu) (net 1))
 (segment (start 106.807 59.817) (end 119.38 59.817) (width 1) (layer F.Cu) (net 2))
 (segment (start 119.38 59.817) (end 119.005 59.817) (width 0.7) (layer B.Cu) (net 2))
 (segment (start 118.993 59.43) (end 119.38 59.817) (width 1) (layer B.Cu) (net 2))
 (segment (start 116.459 59.43) (end 118.993 59.43) (width 1) (layer B.Cu) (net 2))
 (segment (start 112.401 59.43) (end 116.459 59.43) (width 1) (layer B.Cu) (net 2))
 (segment (start 111.76 61.849) (end 111.76 60.071) (width 1) (layer B.Cu) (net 2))
 (segment (start 111.76 60.071) (end 112.401 59.43) (width 1) (layer B.Cu) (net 2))
 (segment (start 106.807 62.357) (end 109.855 62.357) (width 0.7) (layer F.Cu) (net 3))
 (segment (start 110.511999 61.700001) (end 111.884 61.700001) (width 0.7) (layer F.Cu) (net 3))
 (segment (start 109.855 62.357) (end 110.511999 61.700001) (width 0.7) (layer F.Cu) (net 3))
 (segment (start 110.871 64.389) (end 111.884 64.389) (width 0.7) (layer F.Cu) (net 4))
 (segment (start 106.807 64.897) (end 110.363 64.897) (width 0.7) (layer F.Cu) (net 4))
 (segment (start 110.363 64.897) (end 110.871 64.389) (width 0.7) (layer F.Cu) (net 4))
 (segment (start 114.684 64.389) (end 116.586 64.389) (width 0.7) (layer F.Cu) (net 5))
 (segment (start 117.094 64.897) (end 119.38 64.897) (width 0.7) (layer F.Cu) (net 5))
 (segment (start 116.586 64.389) (end 117.094 64.897) (width 0.7) (layer F.Cu) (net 5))
 (segment (start 119.132 64.649) (end 119.38 64.897) (width 1) (layer B.Cu) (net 5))
 (segment (start 111.76 64.649) (end 119.132 64.649) (width 1) (layer B.Cu) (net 5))
 (segment (start 114.684 61.700001) (end 116.691001 61.700001) (width 0.7) (layer F.Cu) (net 6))
 (segment (start 117.348 62.357) (end 119.38 62.357) (width 0.7) (layer F.Cu) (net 6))
 (segment (start 116.691001 61.700001) (end 117.348 62.357) (width 0.7) (layer F.Cu) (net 6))
 (segment (start 119.253 62.23) (end 119.38 62.357) (width 1) (layer B.Cu) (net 6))
 (segment (start 116.459 62.23) (end 119.253 62.23) (width 1) (layer B.Cu) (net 6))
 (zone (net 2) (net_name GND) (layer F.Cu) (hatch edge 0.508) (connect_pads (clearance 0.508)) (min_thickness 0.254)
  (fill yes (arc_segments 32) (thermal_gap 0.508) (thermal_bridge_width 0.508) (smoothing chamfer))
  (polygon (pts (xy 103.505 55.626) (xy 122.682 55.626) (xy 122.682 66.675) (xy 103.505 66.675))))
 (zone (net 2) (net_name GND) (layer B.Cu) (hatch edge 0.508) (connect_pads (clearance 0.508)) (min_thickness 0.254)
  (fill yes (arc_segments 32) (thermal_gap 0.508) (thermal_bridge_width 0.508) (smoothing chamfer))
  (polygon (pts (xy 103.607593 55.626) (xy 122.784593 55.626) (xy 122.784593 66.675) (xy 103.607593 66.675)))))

